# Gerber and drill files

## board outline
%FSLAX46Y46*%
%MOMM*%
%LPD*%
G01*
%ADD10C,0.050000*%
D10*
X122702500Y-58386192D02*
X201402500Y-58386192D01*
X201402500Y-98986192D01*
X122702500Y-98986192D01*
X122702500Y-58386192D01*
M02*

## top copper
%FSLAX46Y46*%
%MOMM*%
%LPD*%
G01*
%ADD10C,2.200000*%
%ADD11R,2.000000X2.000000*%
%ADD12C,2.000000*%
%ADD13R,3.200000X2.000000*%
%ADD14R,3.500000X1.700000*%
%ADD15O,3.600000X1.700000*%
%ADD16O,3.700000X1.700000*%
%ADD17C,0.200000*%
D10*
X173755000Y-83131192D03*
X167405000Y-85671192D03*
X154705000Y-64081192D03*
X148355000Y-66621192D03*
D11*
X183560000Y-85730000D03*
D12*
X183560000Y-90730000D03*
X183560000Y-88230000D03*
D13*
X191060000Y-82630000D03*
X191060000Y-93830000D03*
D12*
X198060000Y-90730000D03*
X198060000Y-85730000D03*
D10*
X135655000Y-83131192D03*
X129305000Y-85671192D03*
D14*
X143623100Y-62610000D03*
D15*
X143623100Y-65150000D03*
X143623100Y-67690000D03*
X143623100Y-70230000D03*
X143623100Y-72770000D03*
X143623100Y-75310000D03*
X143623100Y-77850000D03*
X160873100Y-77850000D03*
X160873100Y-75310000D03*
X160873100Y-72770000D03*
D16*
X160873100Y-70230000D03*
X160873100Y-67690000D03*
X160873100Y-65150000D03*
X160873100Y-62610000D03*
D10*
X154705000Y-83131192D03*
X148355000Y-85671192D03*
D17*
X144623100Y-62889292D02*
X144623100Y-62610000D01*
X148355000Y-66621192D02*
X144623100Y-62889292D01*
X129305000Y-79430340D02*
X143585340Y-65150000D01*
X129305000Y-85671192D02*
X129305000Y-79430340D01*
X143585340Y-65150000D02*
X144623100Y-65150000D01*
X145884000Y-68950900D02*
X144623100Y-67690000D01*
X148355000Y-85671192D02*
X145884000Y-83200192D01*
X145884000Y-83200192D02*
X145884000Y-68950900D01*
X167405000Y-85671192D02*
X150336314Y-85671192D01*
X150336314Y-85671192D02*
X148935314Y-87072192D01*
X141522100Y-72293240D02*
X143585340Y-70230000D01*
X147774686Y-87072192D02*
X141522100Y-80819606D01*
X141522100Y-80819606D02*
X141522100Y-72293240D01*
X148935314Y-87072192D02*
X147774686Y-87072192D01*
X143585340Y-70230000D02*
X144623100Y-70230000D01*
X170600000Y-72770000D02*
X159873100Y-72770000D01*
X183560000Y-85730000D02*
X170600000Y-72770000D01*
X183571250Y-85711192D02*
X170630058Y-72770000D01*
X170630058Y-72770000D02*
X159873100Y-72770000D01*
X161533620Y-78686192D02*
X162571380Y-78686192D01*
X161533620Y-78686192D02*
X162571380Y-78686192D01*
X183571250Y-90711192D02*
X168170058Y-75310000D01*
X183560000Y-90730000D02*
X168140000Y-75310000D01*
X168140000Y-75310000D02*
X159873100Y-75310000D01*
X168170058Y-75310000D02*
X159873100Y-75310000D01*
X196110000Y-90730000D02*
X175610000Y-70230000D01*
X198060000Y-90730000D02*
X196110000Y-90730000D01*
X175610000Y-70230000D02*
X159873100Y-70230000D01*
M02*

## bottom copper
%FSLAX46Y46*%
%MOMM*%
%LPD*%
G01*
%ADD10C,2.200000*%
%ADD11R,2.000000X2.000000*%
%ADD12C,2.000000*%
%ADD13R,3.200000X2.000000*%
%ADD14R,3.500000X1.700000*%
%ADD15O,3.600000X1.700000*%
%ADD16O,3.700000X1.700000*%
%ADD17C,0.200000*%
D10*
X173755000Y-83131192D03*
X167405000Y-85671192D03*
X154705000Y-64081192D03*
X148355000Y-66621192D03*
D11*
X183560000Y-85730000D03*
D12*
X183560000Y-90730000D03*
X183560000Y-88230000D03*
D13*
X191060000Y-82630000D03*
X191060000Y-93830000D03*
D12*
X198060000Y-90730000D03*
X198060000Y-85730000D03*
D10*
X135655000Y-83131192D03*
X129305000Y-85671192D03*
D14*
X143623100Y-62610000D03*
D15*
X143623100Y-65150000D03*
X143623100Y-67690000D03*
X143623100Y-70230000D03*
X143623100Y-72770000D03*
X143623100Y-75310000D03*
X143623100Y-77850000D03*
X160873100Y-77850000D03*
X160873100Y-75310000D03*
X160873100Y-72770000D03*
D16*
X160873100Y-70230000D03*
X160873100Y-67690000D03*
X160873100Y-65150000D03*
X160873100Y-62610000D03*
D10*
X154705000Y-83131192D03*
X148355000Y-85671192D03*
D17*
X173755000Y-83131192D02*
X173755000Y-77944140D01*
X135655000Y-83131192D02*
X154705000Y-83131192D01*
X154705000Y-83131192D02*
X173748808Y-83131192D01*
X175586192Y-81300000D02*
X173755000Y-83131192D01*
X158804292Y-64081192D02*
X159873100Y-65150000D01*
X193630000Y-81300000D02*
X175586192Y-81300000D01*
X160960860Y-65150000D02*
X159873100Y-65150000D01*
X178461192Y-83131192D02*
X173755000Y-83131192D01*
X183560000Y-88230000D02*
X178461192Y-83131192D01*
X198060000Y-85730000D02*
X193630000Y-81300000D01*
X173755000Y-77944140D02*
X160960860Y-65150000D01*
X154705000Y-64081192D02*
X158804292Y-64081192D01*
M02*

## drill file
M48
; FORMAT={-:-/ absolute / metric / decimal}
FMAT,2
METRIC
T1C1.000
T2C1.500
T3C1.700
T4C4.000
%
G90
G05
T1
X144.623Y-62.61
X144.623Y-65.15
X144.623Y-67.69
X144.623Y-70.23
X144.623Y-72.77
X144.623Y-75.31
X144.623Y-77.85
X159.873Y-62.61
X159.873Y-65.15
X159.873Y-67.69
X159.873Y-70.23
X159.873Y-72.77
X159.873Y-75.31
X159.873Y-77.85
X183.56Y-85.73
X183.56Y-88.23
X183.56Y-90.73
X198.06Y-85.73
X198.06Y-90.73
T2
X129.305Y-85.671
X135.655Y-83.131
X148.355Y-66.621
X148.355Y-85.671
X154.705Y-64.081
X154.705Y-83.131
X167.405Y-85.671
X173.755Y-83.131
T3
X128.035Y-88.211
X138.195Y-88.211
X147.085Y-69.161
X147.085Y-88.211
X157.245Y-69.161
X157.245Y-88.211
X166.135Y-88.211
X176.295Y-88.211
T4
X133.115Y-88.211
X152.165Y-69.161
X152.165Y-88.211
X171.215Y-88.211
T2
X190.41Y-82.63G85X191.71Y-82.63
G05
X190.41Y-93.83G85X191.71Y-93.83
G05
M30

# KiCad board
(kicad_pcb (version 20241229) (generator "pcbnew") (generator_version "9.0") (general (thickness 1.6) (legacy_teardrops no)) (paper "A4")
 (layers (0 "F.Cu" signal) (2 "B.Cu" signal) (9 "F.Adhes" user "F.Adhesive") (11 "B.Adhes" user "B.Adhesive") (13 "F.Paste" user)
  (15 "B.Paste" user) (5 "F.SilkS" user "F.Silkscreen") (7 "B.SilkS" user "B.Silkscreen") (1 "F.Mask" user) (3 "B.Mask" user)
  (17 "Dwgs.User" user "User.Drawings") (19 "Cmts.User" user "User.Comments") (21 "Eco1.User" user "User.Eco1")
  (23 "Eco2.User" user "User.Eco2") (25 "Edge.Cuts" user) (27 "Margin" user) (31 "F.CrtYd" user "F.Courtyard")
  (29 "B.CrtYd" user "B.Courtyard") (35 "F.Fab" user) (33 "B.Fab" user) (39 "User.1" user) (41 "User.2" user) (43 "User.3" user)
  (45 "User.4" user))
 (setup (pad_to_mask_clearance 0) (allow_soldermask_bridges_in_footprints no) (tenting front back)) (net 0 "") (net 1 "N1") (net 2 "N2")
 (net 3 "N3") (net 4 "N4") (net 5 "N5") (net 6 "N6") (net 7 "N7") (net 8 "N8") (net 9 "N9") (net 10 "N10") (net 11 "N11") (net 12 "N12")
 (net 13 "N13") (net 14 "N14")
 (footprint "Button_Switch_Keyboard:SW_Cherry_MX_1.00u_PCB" (layer "F.Cu") (at 173.755 83.131192)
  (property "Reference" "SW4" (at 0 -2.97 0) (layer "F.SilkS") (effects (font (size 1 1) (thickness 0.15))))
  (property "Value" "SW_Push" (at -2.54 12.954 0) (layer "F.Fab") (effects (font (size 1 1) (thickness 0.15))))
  (pad "" np_thru_hole circle (at -7.62 5.08) (size 1.7 1.7) (drill 1.7) (layers "*.Cu" "*.Mask"))
  (pad "" np_thru_hole circle (at -2.54 5.08) (size 4 4) (drill 4) (layers "*.Cu" "*.Mask"))
  (pad "" np_thru_hole circle (at 2.54 5.08) (size 1.7 1.7) (drill 1.7) (layers "*.Cu" "*.Mask"))
  (pad "1" thru_hole circle (at 0 0) (size 2.2 2.2) (drill 1.5) (layers "*.Cu" "*.Mask") (remove_unused_layers no) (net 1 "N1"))
  (pad "2" thru_hole circle (at -6.35 2.54) (size 2.2 2.2) (drill 1.5) (layers "*.Cu" "*.Mask") (remove_unused_layers no) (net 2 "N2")))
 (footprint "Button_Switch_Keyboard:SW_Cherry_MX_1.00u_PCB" (layer "F.Cu") (at 154.705 64.081192)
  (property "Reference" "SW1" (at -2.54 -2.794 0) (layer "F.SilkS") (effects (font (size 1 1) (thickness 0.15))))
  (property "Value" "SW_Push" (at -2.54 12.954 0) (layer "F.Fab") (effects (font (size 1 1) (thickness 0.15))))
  (pad "" np_thru_hole circle (at -7.62 5.08) (size 1.7 1.7) (drill 1.7) (layers "*.Cu" "*.Mask"))
  (pad "" np_thru_hole circle (at -2.54 5.08) (size 4 4) (drill 4) (layers "*.Cu" "*.Mask"))
  (pad "" np_thru_hole circle (at 2.54 5.08) (size 1.7 1.7) (drill 1.7) (layers "*.Cu" "*.Mask"))
  (pad "1" thru_hole circle (at 0 0) (size 2.2 2.2) (drill 1.5) (layers "*.Cu" "*.Mask") (remove_unused_layers no) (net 1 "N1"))
  (pad "2" thru_hole circle (at -6.35 2.54) (size 2.2 2.2) (drill 1.5) (layers "*.Cu" "*.Mask") (remove_unused_layers no) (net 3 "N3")))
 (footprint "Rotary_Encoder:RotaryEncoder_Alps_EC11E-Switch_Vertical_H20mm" (layer "F.Cu") (at 183.56 85.73)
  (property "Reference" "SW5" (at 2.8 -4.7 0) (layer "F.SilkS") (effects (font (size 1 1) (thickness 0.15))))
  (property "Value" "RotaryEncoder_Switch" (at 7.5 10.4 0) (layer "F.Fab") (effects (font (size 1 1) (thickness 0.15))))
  (pad "A" thru_hole rect (at 0 0) (size 2 2) (drill 1) (layers "*.Cu" "*.Mask") (remove_unused_layers no) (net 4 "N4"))
  (pad "B" thru_hole circle (at 0 5) (size 2 2) (drill 1) (layers "*.Cu" "*.Mask") (remove_unused_layers no) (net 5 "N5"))
  (pad "C" thru_hole circle (at 0 2.5) (size 2 2) (drill 1) (layers "*.Cu" "*.Mask") (remove_unused_layers no) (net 1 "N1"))
  (pad "MP" thru_hole rect (at 7.5 -3.1) (size 3.2 2) (drill oval 2.8 1.5) (layers "*.Cu" "*.Mask") (remove_unused_layers no))
  (pad "MP" thru_hole rect (at 7.5 8.1) (size 3.2 2) (drill oval 2.8 1.5) (layers "*.Cu" "*.Mask") (remove_unused_layers no))
  (pad "S1" thru_hole circle (at 14.5 5) (size 2 2) (drill 1) (layers "*.Cu" "*.Mask") (remove_unused_layers no) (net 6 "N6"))
  (pad "S2" thru_hole circle (at 14.5 0) (size 2 2) (drill 1) (layers "*.Cu" "*.Mask") (remove_unused_layers no) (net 1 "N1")))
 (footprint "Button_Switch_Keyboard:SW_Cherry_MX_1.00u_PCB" (layer "F.Cu") (at 135.655 83.131192)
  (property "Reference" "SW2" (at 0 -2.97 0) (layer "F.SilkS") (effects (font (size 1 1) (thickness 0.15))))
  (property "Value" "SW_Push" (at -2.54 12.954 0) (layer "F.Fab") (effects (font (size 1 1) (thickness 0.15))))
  (pad "" np_thru_hole circle (at -7.62 5.08) (size 1.7 1.7) (drill 1.7) (layers "*.Cu" "*.Mask"))
  (pad "" np_thru_hole circle (at -2.54 5.08) (size 4 4) (drill 4) (layers "*.Cu" "*.Mask"))
  (pad "" np_thru_hole circle (at 2.54 5.08) (size 1.7 1.7) (drill 1.7) (layers "*.Cu" "*.Mask"))
  (pad "1" thru_hole circle (at 0 0) (size 2.2 2.2) (drill 1.5) (layers "*.Cu" "*.Mask") (remove_unused_layers no) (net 1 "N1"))
  (pad "2" thru_hole circle (at -6.35 2.54) (size 2.2 2.2) (drill 1.5) (layers "*.Cu" "*.Mask") (remove_unused_layers no) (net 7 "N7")))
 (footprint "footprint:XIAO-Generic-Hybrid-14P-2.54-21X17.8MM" (layer "F.Cu") (at 152.2481 70.23)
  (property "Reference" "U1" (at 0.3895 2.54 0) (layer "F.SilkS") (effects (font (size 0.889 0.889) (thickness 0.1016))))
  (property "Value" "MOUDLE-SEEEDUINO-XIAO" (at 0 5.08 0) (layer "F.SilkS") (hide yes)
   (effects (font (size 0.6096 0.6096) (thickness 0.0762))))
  (pad "1" thru_hole rect (at -7.625 -7.62) (size 3.5 1.7) (drill 1 (offset -1 0)) (layers "*.Cu" "*.Mask") (remove_unused_layers no)
   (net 3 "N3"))
  (pad "2" thru_hole oval (at -7.625 -5.08) (size 3.6 1.7) (drill 1 (offset -1 0)) (layers "*.Cu" "*.Mask") (remove_unused_layers no)
   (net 7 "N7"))
  (pad "3" thru_hole oval (at -7.625 -2.54) (size 3.6 1.7) (drill 1 (offset -1 0)) (layers "*.Cu" "*.Mask") (remove_unused_layers no)
   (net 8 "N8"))
  (pad "4" thru_hole oval (at -7.625 0) (size 3.6 1.7) (drill 1 (offset -1 0)) (layers "*.Cu" "*.Mask") (remove_unused_layers no)
   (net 2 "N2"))
  (pad "5" thru_hole oval (at -7.625 2.54) (size 3.6 1.7) (drill 1 (offset -1 0)) (layers "*.Cu" "*.Mask") (remove_unused_layers no)
   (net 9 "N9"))
  (pad "6" thru_hole oval (at -7.625 5.08 180) (size 3.6 1.7) (drill 1 (offset 1 0)) (layers "*.Cu" "*.Mask") (remove_unused_layers no)
   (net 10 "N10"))
  (pad "7" thru_hole oval (at -7.625 7.62) (size 3.6 1.7) (drill 1 (offset -1 0)) (layers "*.Cu" "*.Mask") (remove_unused_layers no)
   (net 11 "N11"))
  (pad "8" thru_hole oval (at 7.625 7.62) (size 3.6 1.7) (drill 1 (offset 1 0)) (layers "*.Cu" "*.Mask") (remove_unused_layers no)
   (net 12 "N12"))
  (pad "9" thru_hole oval (at 7.625 5.08) (size 3.6 1.7) (drill 1 (offset 1 0)) (layers "*.Cu" "*.Mask") (remove_unused_layers no)
   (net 5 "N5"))
  (pad "10" thru_hole oval (at 7.625 2.54) (size 3.6 1.7) (drill 1 (offset 1 0)) (layers "*.Cu" "*.Mask") (remove_unused_layers no)
   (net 4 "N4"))
  (pad "11" thru_hole oval (at 7.625 0) (size 3.7 1.7) (drill 1 (offset 1 0)) (layers "*.Cu" "*.Mask") (remove_unused_layers no)
   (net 6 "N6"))
  (pad "12" thru_hole oval (at 7.625 -2.54) (size 3.7 1.7) (drill 1 (offset 1 0)) (layers "*.Cu" "*.Mask") (remove_unused_layers no)
   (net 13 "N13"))
  (pad "13" thru_hole oval (at 7.625 -5.08) (size 3.7 1.7) (drill 1 (offset 1 0)) (layers "*.Cu" "*.Mask") (remove_unused_layers no)
   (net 1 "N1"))
  (pad "14" thru_hole oval (at 7.625 -7.62) (size 3.7 1.7) (drill 1 (offset 1 0)) (layers "*.Cu" "*.Mask") (remove_unused_layers no)
   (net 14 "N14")))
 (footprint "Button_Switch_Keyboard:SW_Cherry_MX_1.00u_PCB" (layer "F.Cu") (at 154.705 83.131192)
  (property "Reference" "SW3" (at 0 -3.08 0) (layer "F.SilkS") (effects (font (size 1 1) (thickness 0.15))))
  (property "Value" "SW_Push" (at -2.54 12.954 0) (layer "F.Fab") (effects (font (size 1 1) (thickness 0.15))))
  (pad "" np_thru_hole circle (at -7.62 5.08) (size 1.7 1.7) (drill 1.7) (layers "*.Cu" "*.Mask"))
  (pad "" np_thru_hole circle (at -2.54 5.08) (size 4 4) (drill 4) (layers "*.Cu" "*.Mask"))
  (pad "" np_thru_hole circle (at 2.54 5.08) (size 1.7 1.7) (drill 1.7) (layers "*.Cu" "*.Mask"))
  (pad "1" thru_hole circle (at 0 0) (size 2.2 2.2) (drill 1.5) (layers "*.Cu" "*.Mask") (remove_unused_layers no) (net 1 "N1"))
  (pad "2" thru_hole circle (at -6.35 2.54) (size 2.2 2.2) (drill 1.5) (layers "*.Cu" "*.Mask") (remove_unused_layers no) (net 8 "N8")))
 (gr_rect (start 122.7025 58.386192) (end 201.4025 98.986192) (stroke (width 0.05) (type default)) (fill no) (layer "Edge.Cuts"))
 (segment (start 173.755 83.131192) (end 173.755 77.94414) (width 0.2) (layer "B.Cu") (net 1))
 (segment (start 135.655 83.131192) (end 154.705 83.131192) (width 0.2) (layer "B.Cu") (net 1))
 (segment (start 154.705 83.131192) (end 173.748808 83.131192) (width 0.2) (layer "B.Cu") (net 1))
 (segment (start 175.586192 81.3) (end 173.755 83.131192) (width 0.2) (layer "B.Cu") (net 1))
 (segment (start 158.804292 64.081192) (end 159.8731 65.15) (width 0.2) (layer "B.Cu") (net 1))
 (segment (start 193.63 81.3) (end 175.586192 81.3) (width 0.2) (layer "B.Cu") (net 1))
 (segment (start 160.96086 65.15) (end 159.8731 65.15) (width 0.2) (layer "B.Cu") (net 1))
 (segment (start 178.461192 83.131192) (end 173.755 83.131192) (width 0.2) (layer "B.Cu") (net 1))
 (segment (start 183.56 88.23) (end 178.461192 83.131192) (width 0.2) (layer "B.Cu") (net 1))
 (segment (start 198.06 85.73) (end 193.63 81.3) (width 0.2) (layer "B.Cu") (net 1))
 (segment (start 173.755 77.94414) (end 160.96086 65.15) (width 0.2) (layer "B.Cu") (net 1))
 (segment (start 154.705 64.081192) (end 158.804292 64.081192) (width 0.2) (layer "B.Cu") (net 1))
 (segment (start 144.6231 62.889292) (end 144.6231 62.61) (width 0.2) (layer "F.Cu") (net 3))
 (segment (start 148.355 66.621192) (end 144.6231 62.889292) (width 0.2) (layer "F.Cu") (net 3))
 (segment (start 129.305 79.43034) (end 143.58534 65.15) (width 0.2) (layer "F.Cu") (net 7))
 (segment (start 129.305 85.671192) (end 129.305 79.43034) (width 0.2) (layer "F.Cu") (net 7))
 (segment (start 143.58534 65.15) (end 144.6231 65.15) (width 0.2) (layer "F.Cu") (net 7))
 (segment (start 145.884 68.9509) (end 144.6231 67.69) (width 0.2) (layer "F.Cu") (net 8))
 (segment (start 148.355 85.671192) (end 145.884 83.200192) (width 0.2) (layer "F.Cu") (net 8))
 (segment (start 145.884 83.200192) (end 145.884 68.9509) (width 0.2) (layer "F.Cu") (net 8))
 (segment (start 167.405 85.671192) (end 150.336314 85.671192) (width 0.2) (layer "F.Cu") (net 2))
 (segment (start 150.336314 85.671192) (end 148.935314 87.072192) (width 0.2) (layer "F.Cu") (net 2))
 (segment (start 141.5221 72.29324) (end 143.58534 70.23) (width 0.2) (layer "F.Cu") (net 2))
 (segment (start 147.774686 87.072192) (end 141.5221 80.819606) (width 0.2) (layer "F.Cu") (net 2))
 (segment (start 141.5221 80.819606) (end 141.5221 72.29324) (width 0.2) (layer "F.Cu") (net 2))
 (segment (start 148.935314 87.072192) (end 147.774686 87.072192) (width 0.2) (layer "F.Cu") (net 2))
 (segment (start 143.58534 70.23) (end 144.6231 70.23) (width 0.2) (layer "F.Cu") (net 2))
 (segment (start 170.6 72.77) (end 159.8731 72.77) (width 0.2) (layer "F.Cu") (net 4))
 (segment (start 183.56 85.73) (end 170.6 72.77) (width 0.2) (layer "F.Cu") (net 4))
 (segment (start 183.57125 85.711192) (end 170.630058 72.77) (width 0.2) (layer "F.Cu") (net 4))
 (segment (start 170.630058 72.77) (end 159.8731 72.77) (width 0.2) (layer "F.Cu") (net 4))
 (segment (start 161.53362 78.686192) (end 162.57138 78.686192) (width 0.2) (layer "F.Cu") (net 12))
 (segment (start 161.53362 78.686192) (end 162.57138 78.686192) (width 0.2) (layer "F.Cu") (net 12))
 (segment (start 183.57125 90.711192) (end 168.170058 75.31) (width 0.2) (layer "F.Cu") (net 5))
 (segment (start 183.56 90.73) (end 168.14 75.31) (width 0.2) (layer "F.Cu") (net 5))
 (segment (start 168.14 75.31) (end 159.8731 75.31) (width 0.2) (layer "F.Cu") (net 5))
 (segment (start 168.170058 75.31) (end 159.8731 75.31) (width 0.2) (layer "F.Cu") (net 5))
 (segment (start 196.11 90.73) (end 175.61 70.23) (width 0.2) (layer "F.Cu") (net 6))
 (segment (start 198.06 90.73) (end 196.11 90.73) (width 0.2) (layer "F.Cu") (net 6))
 (segment (start 175.61 70.23) (end 159.8731 70.23) (width 0.2) (layer "F.Cu") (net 6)))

